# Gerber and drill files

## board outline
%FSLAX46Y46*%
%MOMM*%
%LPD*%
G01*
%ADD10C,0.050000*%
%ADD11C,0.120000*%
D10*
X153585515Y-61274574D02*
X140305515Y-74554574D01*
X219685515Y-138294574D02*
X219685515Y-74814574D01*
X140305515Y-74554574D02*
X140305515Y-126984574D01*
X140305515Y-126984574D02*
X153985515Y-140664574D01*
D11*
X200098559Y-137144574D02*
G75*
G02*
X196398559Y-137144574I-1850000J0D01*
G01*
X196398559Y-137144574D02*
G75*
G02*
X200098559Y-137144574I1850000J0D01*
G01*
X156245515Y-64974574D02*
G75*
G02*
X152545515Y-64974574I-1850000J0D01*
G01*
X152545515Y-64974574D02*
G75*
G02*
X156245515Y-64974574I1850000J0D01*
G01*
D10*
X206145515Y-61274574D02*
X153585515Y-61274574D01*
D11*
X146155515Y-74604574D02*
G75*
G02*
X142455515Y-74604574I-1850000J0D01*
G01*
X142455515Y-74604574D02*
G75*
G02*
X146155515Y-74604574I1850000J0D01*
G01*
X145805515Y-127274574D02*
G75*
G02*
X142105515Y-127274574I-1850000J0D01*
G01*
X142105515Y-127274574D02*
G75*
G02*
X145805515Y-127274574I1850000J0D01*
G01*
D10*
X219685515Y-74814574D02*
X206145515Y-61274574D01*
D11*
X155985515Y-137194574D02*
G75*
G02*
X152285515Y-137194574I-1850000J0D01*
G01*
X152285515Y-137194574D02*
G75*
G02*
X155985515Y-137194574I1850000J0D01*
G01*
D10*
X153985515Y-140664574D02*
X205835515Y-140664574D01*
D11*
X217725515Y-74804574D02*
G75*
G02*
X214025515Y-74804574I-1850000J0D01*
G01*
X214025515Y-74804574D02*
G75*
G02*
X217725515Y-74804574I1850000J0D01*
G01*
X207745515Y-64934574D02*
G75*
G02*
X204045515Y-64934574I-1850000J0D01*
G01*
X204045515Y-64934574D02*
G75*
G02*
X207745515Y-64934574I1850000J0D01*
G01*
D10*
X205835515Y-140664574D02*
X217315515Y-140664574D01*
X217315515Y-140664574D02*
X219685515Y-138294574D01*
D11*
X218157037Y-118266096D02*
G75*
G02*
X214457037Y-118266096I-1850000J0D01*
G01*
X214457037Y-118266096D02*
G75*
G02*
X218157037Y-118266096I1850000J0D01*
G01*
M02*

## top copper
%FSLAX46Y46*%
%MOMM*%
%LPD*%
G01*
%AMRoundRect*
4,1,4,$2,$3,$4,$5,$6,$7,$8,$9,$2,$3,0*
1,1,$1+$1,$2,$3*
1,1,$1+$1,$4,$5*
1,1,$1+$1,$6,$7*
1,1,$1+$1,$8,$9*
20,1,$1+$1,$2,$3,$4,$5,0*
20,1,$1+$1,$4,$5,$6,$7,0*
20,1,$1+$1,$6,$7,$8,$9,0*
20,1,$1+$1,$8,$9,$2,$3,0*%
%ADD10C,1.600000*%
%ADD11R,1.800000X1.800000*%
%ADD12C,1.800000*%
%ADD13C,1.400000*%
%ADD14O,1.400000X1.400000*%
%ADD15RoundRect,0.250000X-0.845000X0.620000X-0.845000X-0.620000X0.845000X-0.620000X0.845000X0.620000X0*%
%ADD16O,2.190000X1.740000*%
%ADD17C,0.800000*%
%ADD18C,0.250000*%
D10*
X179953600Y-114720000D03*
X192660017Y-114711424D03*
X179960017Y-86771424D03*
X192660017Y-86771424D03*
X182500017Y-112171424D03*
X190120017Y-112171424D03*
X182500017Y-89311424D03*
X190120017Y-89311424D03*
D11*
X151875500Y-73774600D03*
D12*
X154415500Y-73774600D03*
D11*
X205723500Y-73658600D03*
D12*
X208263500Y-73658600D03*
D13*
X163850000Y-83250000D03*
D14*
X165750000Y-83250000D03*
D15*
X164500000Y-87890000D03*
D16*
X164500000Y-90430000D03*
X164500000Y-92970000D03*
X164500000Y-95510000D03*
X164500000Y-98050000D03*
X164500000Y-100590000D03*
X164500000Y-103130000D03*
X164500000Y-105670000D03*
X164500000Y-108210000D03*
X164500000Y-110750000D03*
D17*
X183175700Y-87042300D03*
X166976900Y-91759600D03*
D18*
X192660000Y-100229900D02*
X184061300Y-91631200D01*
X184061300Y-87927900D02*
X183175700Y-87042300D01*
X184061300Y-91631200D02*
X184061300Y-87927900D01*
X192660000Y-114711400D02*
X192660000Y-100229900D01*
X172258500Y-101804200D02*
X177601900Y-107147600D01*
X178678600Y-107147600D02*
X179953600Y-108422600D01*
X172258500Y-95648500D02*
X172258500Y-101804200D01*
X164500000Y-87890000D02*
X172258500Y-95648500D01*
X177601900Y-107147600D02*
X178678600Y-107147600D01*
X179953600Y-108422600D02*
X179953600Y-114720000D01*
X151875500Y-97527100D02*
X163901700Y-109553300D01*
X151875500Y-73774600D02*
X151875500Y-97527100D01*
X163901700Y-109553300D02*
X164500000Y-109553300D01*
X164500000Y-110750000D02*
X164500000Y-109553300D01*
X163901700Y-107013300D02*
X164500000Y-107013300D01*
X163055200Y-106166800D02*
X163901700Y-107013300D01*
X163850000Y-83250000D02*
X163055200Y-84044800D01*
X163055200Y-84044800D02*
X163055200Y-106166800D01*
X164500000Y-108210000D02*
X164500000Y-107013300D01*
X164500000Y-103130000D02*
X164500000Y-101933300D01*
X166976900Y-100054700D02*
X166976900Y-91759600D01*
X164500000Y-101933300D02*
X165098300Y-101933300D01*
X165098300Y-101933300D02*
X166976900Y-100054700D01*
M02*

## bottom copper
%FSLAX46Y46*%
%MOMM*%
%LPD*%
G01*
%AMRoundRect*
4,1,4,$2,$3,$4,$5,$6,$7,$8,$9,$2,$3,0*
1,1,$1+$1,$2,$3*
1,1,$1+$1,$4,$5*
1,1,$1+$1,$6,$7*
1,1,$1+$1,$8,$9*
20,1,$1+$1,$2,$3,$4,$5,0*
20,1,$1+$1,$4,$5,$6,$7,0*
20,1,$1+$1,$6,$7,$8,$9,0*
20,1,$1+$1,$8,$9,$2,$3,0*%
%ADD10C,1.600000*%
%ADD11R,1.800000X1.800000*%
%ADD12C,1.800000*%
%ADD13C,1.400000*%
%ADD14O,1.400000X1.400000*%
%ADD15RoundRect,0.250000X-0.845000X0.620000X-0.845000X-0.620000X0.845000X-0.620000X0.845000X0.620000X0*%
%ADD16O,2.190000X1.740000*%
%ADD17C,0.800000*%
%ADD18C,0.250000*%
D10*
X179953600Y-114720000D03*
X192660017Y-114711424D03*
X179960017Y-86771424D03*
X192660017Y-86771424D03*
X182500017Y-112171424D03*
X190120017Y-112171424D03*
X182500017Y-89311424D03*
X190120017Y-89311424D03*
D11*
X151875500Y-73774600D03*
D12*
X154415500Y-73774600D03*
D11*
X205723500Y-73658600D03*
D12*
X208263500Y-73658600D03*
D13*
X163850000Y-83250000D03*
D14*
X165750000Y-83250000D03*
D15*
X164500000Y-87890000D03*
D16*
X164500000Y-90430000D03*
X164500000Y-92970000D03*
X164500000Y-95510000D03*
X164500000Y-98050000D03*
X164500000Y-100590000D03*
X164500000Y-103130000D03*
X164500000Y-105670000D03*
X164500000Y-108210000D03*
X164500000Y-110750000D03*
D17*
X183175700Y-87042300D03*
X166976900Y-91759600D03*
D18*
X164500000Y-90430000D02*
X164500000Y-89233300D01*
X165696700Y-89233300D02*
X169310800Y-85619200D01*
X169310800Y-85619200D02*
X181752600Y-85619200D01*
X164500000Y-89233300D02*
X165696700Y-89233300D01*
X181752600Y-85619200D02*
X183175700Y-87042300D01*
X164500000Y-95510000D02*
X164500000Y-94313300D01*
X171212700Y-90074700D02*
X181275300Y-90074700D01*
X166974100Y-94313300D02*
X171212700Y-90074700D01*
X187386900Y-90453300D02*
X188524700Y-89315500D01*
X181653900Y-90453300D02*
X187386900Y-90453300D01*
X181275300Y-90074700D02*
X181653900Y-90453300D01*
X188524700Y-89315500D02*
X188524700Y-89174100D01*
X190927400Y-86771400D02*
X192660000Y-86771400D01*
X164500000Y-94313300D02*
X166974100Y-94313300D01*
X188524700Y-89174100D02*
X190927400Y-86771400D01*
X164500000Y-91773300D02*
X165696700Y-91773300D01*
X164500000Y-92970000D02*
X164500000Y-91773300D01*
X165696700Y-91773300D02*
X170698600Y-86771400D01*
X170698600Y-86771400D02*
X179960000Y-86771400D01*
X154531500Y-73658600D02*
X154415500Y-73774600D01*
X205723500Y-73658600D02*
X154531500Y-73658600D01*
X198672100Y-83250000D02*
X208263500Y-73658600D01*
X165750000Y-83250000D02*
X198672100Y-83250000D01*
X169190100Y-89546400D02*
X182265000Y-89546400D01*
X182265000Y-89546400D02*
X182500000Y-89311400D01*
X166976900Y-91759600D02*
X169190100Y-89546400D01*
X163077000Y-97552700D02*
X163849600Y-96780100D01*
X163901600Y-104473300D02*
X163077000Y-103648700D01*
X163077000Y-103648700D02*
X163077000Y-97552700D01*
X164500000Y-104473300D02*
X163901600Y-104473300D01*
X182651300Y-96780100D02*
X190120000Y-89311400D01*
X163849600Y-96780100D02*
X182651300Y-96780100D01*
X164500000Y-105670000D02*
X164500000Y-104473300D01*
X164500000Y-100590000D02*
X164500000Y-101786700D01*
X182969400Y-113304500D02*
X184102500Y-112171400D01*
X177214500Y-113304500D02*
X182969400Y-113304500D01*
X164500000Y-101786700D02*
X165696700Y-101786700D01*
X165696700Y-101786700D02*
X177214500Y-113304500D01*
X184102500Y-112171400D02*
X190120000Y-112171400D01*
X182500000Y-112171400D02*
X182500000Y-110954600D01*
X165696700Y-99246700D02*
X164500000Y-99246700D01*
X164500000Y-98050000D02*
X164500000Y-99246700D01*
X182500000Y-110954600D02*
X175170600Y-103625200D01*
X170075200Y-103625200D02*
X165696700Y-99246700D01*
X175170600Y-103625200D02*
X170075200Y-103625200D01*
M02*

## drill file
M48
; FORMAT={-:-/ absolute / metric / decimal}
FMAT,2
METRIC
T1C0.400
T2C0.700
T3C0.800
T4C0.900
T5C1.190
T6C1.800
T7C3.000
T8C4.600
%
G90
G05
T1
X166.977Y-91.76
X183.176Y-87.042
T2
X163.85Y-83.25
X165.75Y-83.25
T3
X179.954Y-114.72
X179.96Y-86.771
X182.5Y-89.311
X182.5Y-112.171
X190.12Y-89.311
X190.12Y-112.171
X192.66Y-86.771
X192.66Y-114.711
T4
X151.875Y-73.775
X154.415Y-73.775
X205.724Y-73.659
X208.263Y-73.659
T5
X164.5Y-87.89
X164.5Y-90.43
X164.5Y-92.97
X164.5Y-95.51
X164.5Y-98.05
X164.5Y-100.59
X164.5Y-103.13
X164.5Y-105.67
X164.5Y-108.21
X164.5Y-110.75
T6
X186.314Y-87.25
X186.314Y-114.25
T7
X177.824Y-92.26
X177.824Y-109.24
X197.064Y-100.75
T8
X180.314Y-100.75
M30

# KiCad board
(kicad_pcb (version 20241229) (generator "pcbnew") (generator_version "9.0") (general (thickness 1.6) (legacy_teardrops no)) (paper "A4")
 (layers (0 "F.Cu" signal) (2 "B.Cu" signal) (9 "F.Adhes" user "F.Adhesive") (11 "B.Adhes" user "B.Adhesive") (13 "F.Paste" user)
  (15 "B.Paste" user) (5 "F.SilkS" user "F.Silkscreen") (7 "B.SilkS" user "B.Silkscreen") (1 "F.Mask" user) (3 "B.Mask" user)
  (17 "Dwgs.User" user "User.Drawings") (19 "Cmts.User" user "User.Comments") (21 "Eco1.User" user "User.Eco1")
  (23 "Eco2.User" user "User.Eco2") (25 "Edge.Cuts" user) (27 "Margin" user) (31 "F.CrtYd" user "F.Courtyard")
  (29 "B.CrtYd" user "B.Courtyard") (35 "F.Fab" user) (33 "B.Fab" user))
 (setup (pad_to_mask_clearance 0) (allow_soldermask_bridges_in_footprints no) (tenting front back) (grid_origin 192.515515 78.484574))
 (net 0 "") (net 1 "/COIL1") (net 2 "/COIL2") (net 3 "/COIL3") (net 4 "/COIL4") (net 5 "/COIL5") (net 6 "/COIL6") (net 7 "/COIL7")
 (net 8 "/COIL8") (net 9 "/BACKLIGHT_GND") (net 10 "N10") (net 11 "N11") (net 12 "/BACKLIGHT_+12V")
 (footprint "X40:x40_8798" (layer "F.Cu") (at 186.3136 100.75 90)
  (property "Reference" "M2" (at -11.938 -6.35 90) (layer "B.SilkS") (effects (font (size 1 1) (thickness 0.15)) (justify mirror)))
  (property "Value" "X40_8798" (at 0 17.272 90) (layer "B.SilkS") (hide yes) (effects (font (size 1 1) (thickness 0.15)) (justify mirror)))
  (pad "" np_thru_hole circle (at -13.5 0 90) (size 1.8 1.8) (drill 1.8) (layers "*.Cu" "*.Mask"))
  (pad "" np_thru_hole circle (at -8.49 -8.49 90) (size 3 3) (drill 3) (layers "*.Cu" "*.Mask"))
  (pad "" np_thru_hole circle (at 0 -6 90) (size 4.6 4.6) (drill 4.6) (layers "*.Cu" "*.Mask"))
  (pad "" np_thru_hole circle (at 0 10.75 90) (size 3 3) (drill 3) (layers "*.Cu" "*.Mask"))
  (pad "" np_thru_hole circle (at 8.49 -8.49 90) (size 3 3) (drill 3) (layers "*.Cu" "*.Mask"))
  (pad "" np_thru_hole circle (at 13.5 0 90) (size 1.8 1.8) (drill 1.8) (layers "*.Cu" "*.Mask"))
  (pad "1" thru_hole circle (at -13.97 -6.36 90) (size 1.6 1.6) (drill 0.8) (layers "*.Cu" "*.Mask") (remove_unused_layers no)
   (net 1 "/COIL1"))
  (pad "2" thru_hole circle (at -13.961424 6.346417 90) (size 1.6 1.6) (drill 0.8) (layers "*.Cu" "*.Mask") (remove_unused_layers no)
   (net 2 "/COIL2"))
  (pad "3" thru_hole circle (at 13.978576 -6.353583 90) (size 1.6 1.6) (drill 0.8) (layers "*.Cu" "*.Mask") (remove_unused_layers no)
   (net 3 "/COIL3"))
  (pad "4" thru_hole circle (at 13.978576 6.346417 90) (size 1.6 1.6) (drill 0.8) (layers "*.Cu" "*.Mask") (remove_unused_layers no)
   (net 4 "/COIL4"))
  (pad "5" thru_hole circle (at -11.421424 -3.813583 90) (size 1.6 1.6) (drill 0.8) (layers "*.Cu" "*.Mask") (remove_unused_layers no)
   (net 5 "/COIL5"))
  (pad "6" thru_hole circle (at -11.421424 3.806417 90) (size 1.6 1.6) (drill 0.8) (layers "*.Cu" "*.Mask") (remove_unused_layers no)
   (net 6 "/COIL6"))
  (pad "7" thru_hole circle (at 11.438576 -3.813583 90) (size 1.6 1.6) (drill 0.8) (layers "*.Cu" "*.Mask") (remove_unused_layers no)
   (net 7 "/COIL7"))
  (pad "8" thru_hole circle (at 11.438576 3.806417 90) (size 1.6 1.6) (drill 0.8) (layers "*.Cu" "*.Mask") (remove_unused_layers no)
   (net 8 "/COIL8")))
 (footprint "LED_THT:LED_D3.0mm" (layer "F.Cu") (at 151.8755 73.7746)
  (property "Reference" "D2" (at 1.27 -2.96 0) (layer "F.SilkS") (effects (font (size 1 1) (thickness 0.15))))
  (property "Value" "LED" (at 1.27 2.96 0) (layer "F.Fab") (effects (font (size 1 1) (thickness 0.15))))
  (pad "1" thru_hole rect (at 0 0) (size 1.8 1.8) (drill 0.9) (layers "*.Cu" "*.Mask") (remove_unused_layers no) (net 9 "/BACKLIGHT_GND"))
  (pad "2" thru_hole circle (at 2.54 0) (size 1.8 1.8) (drill 0.9) (layers "*.Cu" "*.Mask") (remove_unused_layers no) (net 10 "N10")))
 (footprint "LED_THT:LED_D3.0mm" (layer "F.Cu") (at 205.7235 73.6586)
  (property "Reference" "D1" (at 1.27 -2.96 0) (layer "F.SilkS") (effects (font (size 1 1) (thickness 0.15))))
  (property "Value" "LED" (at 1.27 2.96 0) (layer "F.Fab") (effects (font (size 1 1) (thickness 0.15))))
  (pad "1" thru_hole rect (at 0 0) (size 1.8 1.8) (drill 0.9) (layers "*.Cu" "*.Mask") (remove_unused_layers no) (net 10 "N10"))
  (pad "2" thru_hole circle (at 2.54 0) (size 1.8 1.8) (drill 0.9) (layers "*.Cu" "*.Mask") (remove_unused_layers no) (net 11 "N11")))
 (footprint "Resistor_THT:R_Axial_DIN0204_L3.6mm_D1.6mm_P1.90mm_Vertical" (layer "B.Cu") (at 163.85 83.25)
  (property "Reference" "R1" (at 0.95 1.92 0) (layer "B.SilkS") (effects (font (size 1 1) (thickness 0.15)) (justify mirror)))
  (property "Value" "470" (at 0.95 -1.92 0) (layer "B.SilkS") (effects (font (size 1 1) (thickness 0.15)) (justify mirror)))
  (pad "1" thru_hole circle (at 0 0) (size 1.4 1.4) (drill 0.7) (layers "*.Cu" "*.Mask") (remove_unused_layers no)
   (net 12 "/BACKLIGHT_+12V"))
  (pad "2" thru_hole oval (at 1.9 0) (size 1.4 1.4) (drill 0.7) (layers "*.Cu" "*.Mask") (remove_unused_layers no) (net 11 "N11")))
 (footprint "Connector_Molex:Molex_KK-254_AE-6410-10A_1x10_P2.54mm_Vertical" (layer "B.Cu") (at 164.5 87.89 -90)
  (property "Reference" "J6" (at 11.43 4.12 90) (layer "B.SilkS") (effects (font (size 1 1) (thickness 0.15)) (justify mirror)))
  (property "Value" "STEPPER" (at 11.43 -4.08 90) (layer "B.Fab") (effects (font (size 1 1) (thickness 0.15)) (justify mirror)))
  (pad "1" thru_hole roundrect (at 0 0 270) (size 1.74 2.19) (drill 1.19) (layers "*.Cu" "*.Mask") (remove_unused_layers no)
   (roundrect_rratio 0.143678) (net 1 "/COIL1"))
  (pad "2" thru_hole oval (at 2.54 0 270) (size 1.74 2.19) (drill 1.19) (layers "*.Cu" "*.Mask") (remove_unused_layers no) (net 2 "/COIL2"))
  (pad "3" thru_hole oval (at 5.08 0 270) (size 1.74 2.19) (drill 1.19) (layers "*.Cu" "*.Mask") (remove_unused_layers no) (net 3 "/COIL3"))
  (pad "4" thru_hole oval (at 7.62 0 270) (size 1.74 2.19) (drill 1.19) (layers "*.Cu" "*.Mask") (remove_unused_layers no) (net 4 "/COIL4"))
  (pad "5" thru_hole oval (at 10.16 0 270) (size 1.74 2.19) (drill 1.19) (layers "*.Cu" "*.Mask") (remove_unused_layers no) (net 5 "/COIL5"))
  (pad "6" thru_hole oval (at 12.7 0 270) (size 1.74 2.19) (drill 1.19) (layers "*.Cu" "*.Mask") (remove_unused_layers no) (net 6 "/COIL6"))
  (pad "7" thru_hole oval (at 15.24 0 270) (size 1.74 2.19) (drill 1.19) (layers "*.Cu" "*.Mask") (remove_unused_layers no) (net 7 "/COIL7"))
  (pad "8" thru_hole oval (at 17.78 0 270) (size 1.74 2.19) (drill 1.19) (layers "*.Cu" "*.Mask") (remove_unused_layers no) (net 8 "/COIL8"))
  (pad "9" thru_hole oval (at 20.32 0 270) (size 1.74 2.19) (drill 1.19) (layers "*.Cu" "*.Mask") (remove_unused_layers no)
   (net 12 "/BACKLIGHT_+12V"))
  (pad "10" thru_hole oval (at 22.86 0 270) (size 1.74 2.19) (drill 1.19) (layers "*.Cu" "*.Mask") (remove_unused_layers no)
   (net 9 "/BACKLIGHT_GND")))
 (gr_line (start 153.585515 61.274574) (end 140.305515 74.554574) (stroke (width 0.05) (type solid)) (layer "Edge.Cuts"))
 (gr_line (start 219.685515 138.294574) (end 219.685515 74.814574) (stroke (width 0.05) (type solid)) (layer "Edge.Cuts"))
 (gr_line (start 140.305515 74.554574) (end 140.305515 126.984574) (stroke (width 0.05) (type solid)) (layer "Edge.Cuts"))
 (gr_line (start 140.305515 126.984574) (end 153.985515 140.664574) (stroke (width 0.05) (type solid)) (layer "Edge.Cuts"))
 (gr_circle (center 198.248559 137.144574) (end 200.098559 137.144574) (stroke (width 0.12) (type solid)) (fill no) (layer "Edge.Cuts"))
 (gr_circle (center 154.395515 64.974574) (end 156.245515 64.974574) (stroke (width 0.12) (type solid)) (fill no) (layer "Edge.Cuts"))
 (gr_line (start 206.145515 61.274574) (end 153.585515 61.274574) (stroke (width 0.05) (type solid)) (layer "Edge.Cuts"))
 (gr_circle (center 144.305515 74.604574) (end 146.155515 74.604574) (stroke (width 0.12) (type solid)) (fill no) (layer "Edge.Cuts"))
 (gr_circle (center 143.955515 127.274574) (end 145.805515 127.274574) (stroke (width 0.12) (type solid)) (fill no) (layer "Edge.Cuts"))
 (gr_line (start 219.685515 74.814574) (end 206.145515 61.274574) (stroke (width 0.05) (type solid)) (layer "Edge.Cuts"))
 (gr_circle (center 154.135515 137.194574) (end 155.985515 137.194574) (stroke (width 0.12) (type solid)) (fill no) (layer "Edge.Cuts"))
 (gr_line (start 153.985515 140.664574) (end 205.835515 140.664574) (stroke (width 0.05) (type solid)) (layer "Edge.Cuts"))
 (gr_circle (center 215.875515 74.804574) (end 217.725515 74.804574) (stroke (width 0.12) (type solid)) (fill no) (layer "Edge.Cuts"))
 (gr_circle (center 205.895515 64.934574) (end 207.745515 64.934574) (stroke (width 0.12) (type solid)) (fill no) (layer "Edge.Cuts"))
 (gr_line (start 205.835515 140.664574) (end 217.315515 140.664574) (stroke (width 0.05) (type solid)) (layer "Edge.Cuts"))
 (gr_line (start 217.315515 140.664574) (end 219.685515 138.294574) (stroke (width 0.05) (type solid)) (layer "Edge.Cuts"))
 (gr_circle (center 216.307037 118.266096) (end 218.157037 118.266096) (stroke (width 0.12) (type solid)) (fill no) (layer "Edge.Cuts"))
 (segment (start 192.66 100.2299) (end 184.0613 91.6312) (width 0.25) (layer "F.Cu") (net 2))
 (segment (start 184.0613 87.9279) (end 183.1757 87.0423) (width 0.25) (layer "F.Cu") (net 2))
 (segment (start 184.0613 91.6312) (end 184.0613 87.9279) (width 0.25) (layer "F.Cu") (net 2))
 (segment (start 192.66 114.7114) (end 192.66 100.2299) (width 0.25) (layer "F.Cu") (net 2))
 (via (at 183.1757 87.0423) (size 0.8) (drill 0.4) (layers "F.Cu" "B.Cu") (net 2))
 (segment (start 164.5 90.43) (end 164.5 89.2333) (width 0.25) (layer "B.Cu") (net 2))
 (segment (start 165.6967 89.2333) (end 169.3108 85.6192) (width 0.25) (layer "B.Cu") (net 2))
 (segment (start 169.3108 85.6192) (end 181.7526 85.6192) (width 0.25) (layer "B.Cu") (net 2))
 (segment (start 164.5 89.2333) (end 165.6967 89.2333) (width 0.25) (layer "B.Cu") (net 2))
 (segment (start 181.7526 85.6192) (end 183.1757 87.0423) (width 0.25) (layer "B.Cu") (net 2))
 (segment (start 172.2585 101.8042) (end 177.6019 107.1476) (width 0.25) (layer "F.Cu") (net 1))
 (segment (start 178.6786 107.1476) (end 179.9536 108.4226) (width 0.25) (layer "F.Cu") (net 1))
 (segment (start 172.2585 95.6485) (end 172.2585 101.8042) (width 0.25) (layer "F.Cu") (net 1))
 (segment (start 164.5 87.89) (end 172.2585 95.6485) (width 0.25) (layer "F.Cu") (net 1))
 (segment (start 177.6019 107.1476) (end 178.6786 107.1476) (width 0.25) (layer "F.Cu") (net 1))
 (segment (start 179.9536 108.4226) (end 179.9536 114.72) (width 0.25) (layer "F.Cu") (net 1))
 (segment (start 164.5 95.51) (end 164.5 94.3133) (width 0.25) (layer "B.Cu") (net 4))
 (segment (start 171.2127 90.0747) (end 181.2753 90.0747) (width 0.25) (layer "B.Cu") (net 4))
 (segment (start 166.9741 94.3133) (end 171.2127 90.0747) (width 0.25) (layer "B.Cu") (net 4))
 (segment (start 187.3869 90.4533) (end 188.5247 89.3155) (width 0.25) (layer "B.Cu") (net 4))
 (segment (start 181.6539 90.4533) (end 187.3869 90.4533) (width 0.25) (layer "B.Cu") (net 4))
 (segment (start 181.2753 90.0747) (end 181.6539 90.4533) (width 0.25) (layer "B.Cu") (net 4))
 (segment (start 188.5247 89.3155) (end 188.5247 89.1741) (width 0.25) (layer "B.Cu") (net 4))
 (segment (start 190.9274 86.7714) (end 192.66 86.7714) (width 0.25) (layer "B.Cu") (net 4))
 (segment (start 164.5 94.3133) (end 166.9741 94.3133) (width 0.25) (layer "B.Cu") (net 4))
 (segment (start 188.5247 89.1741) (end 190.9274 86.7714) (width 0.25) (layer "B.Cu") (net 4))
 (segment (start 164.5 91.7733) (end 165.6967 91.7733) (width 0.25) (layer "B.Cu") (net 3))
 (segment (start 164.5 92.97) (end 164.5 91.7733) (width 0.25) (layer "B.Cu") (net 3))
 (segment (start 165.6967 91.7733) (end 170.6986 86.7714) (width 0.25) (layer "B.Cu") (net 3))
 (segment (start 170.6986 86.7714) (end 179.96 86.7714) (width 0.25) (layer "B.Cu") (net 3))
 (segment (start 154.5315 73.6586) (end 154.4155 73.7746) (width 0.25) (layer "B.Cu") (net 10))
 (segment (start 205.7235 73.6586) (end 154.5315 73.6586) (width 0.25) (layer "B.Cu") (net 10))
 (segment (start 198.6721 83.25) (end 208.2635 73.6586) (width 0.25) (layer "B.Cu") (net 11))
 (segment (start 165.75 83.25) (end 198.6721 83.25) (width 0.25) (layer "B.Cu") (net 11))
 (segment (start 151.8755 97.5271) (end 163.9017 109.5533) (width 0.25) (layer "F.Cu") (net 9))
 (segment (start 151.8755 73.7746) (end 151.8755 97.5271) (width 0.25) (layer "F.Cu") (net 9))
 (segment (start 163.9017 109.5533) (end 164.5 109.5533) (width 0.25) (layer "F.Cu") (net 9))
 (segment (start 164.5 110.75) (end 164.5 109.5533) (width 0.25) (layer "F.Cu") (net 9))
 (segment (start 163.9017 107.0133) (end 164.5 107.0133) (width 0.25) (layer "F.Cu") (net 12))
 (segment (start 163.0552 106.1668) (end 163.9017 107.0133) (width 0.25) (layer "F.Cu") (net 12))
 (segment (start 163.85 83.25) (end 163.0552 84.0448) (width 0.25) (layer "F.Cu") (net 12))
 (segment (start 163.0552 84.0448) (end 163.0552 106.1668) (width 0.25) (layer "F.Cu") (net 12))
 (segment (start 164.5 108.21) (end 164.5 107.0133) (width 0.25) (layer "F.Cu") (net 12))
 (segment (start 164.5 103.13) (end 164.5 101.9333) (width 0.25) (layer "F.Cu") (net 7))
 (segment (start 166.9769 100.0547) (end 166.9769 91.7596) (width 0.25) (layer "F.Cu") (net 7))
 (segment (start 164.5 101.9333) (end 165.0983 101.9333) (width 0.25) (layer "F.Cu") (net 7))
 (segment (start 165.0983 101.9333) (end 166.9769 100.0547) (width 0.25) (layer "F.Cu") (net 7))
 (via (at 166.9769 91.7596) (size 0.8) (drill 0.4) (layers "F.Cu" "B.Cu") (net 7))
 (segment (start 169.1901 89.5464) (end 182.265 89.5464) (width 0.25) (layer "B.Cu") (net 7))
 (segment (start 182.265 89.5464) (end 182.5 89.3114) (width 0.25) (layer "B.Cu") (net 7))
 (segment (start 166.9769 91.7596) (end 169.1901 89.5464) (width 0.25) (layer "B.Cu") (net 7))
 (segment (start 163.077 97.5527) (end 163.8496 96.7801) (width 0.25) (layer "B.Cu") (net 8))
 (segment (start 163.9016 104.4733) (end 163.077 103.6487) (width 0.25) (layer "B.Cu") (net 8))
 (segment (start 163.077 103.6487) (end 163.077 97.5527) (width 0.25) (layer "B.Cu") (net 8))
 (segment (start 164.5 104.4733) (end 163.9016 104.4733) (width 0.25) (layer "B.Cu") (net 8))
 (segment (start 182.6513 96.7801) (end 190.12 89.3114) (width 0.25) (layer "B.Cu") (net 8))
 (segment (start 163.8496 96.7801) (end 182.6513 96.7801) (width 0.25) (layer "B.Cu") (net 8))
 (segment (start 164.5 105.67) (end 164.5 104.4733) (width 0.25) (layer "B.Cu") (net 8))
 (segment (start 164.5 100.59) (end 164.5 101.7867) (width 0.25) (layer "B.Cu") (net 6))
 (segment (start 182.9694 113.3045) (end 184.1025 112.1714) (width 0.25) (layer "B.Cu") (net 6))
 (segment (start 177.2145 113.3045) (end 182.9694 113.3045) (width 0.25) (layer "B.Cu") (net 6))
 (segment (start 164.5 101.7867) (end 165.6967 101.7867) (width 0.25) (layer "B.Cu") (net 6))
 (segment (start 165.6967 101.7867) (end 177.2145 113.3045) (width 0.25) (layer "B.Cu") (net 6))
 (segment (start 184.1025 112.1714) (end 190.12 112.1714) (width 0.25) (layer "B.Cu") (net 6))
 (segment (start 182.5 112.1714) (end 182.5 110.9546) (width 0.25) (layer "B.Cu") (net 5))
 (segment (start 165.6967 99.2467) (end 164.5 99.2467) (width 0.25) (layer "B.Cu") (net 5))
 (segment (start 164.5 98.05) (end 164.5 99.2467) (width 0.25) (layer "B.Cu") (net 5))
 (segment (start 182.5 110.9546) (end 175.1706 103.6252) (width 0.25) (layer "B.Cu") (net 5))
 (segment (start 170.0752 103.6252) (end 165.6967 99.2467) (width 0.25) (layer "B.Cu") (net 5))
 (segment (start 175.1706 103.6252) (end 170.0752 103.6252) (width 0.25) (layer "B.Cu") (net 5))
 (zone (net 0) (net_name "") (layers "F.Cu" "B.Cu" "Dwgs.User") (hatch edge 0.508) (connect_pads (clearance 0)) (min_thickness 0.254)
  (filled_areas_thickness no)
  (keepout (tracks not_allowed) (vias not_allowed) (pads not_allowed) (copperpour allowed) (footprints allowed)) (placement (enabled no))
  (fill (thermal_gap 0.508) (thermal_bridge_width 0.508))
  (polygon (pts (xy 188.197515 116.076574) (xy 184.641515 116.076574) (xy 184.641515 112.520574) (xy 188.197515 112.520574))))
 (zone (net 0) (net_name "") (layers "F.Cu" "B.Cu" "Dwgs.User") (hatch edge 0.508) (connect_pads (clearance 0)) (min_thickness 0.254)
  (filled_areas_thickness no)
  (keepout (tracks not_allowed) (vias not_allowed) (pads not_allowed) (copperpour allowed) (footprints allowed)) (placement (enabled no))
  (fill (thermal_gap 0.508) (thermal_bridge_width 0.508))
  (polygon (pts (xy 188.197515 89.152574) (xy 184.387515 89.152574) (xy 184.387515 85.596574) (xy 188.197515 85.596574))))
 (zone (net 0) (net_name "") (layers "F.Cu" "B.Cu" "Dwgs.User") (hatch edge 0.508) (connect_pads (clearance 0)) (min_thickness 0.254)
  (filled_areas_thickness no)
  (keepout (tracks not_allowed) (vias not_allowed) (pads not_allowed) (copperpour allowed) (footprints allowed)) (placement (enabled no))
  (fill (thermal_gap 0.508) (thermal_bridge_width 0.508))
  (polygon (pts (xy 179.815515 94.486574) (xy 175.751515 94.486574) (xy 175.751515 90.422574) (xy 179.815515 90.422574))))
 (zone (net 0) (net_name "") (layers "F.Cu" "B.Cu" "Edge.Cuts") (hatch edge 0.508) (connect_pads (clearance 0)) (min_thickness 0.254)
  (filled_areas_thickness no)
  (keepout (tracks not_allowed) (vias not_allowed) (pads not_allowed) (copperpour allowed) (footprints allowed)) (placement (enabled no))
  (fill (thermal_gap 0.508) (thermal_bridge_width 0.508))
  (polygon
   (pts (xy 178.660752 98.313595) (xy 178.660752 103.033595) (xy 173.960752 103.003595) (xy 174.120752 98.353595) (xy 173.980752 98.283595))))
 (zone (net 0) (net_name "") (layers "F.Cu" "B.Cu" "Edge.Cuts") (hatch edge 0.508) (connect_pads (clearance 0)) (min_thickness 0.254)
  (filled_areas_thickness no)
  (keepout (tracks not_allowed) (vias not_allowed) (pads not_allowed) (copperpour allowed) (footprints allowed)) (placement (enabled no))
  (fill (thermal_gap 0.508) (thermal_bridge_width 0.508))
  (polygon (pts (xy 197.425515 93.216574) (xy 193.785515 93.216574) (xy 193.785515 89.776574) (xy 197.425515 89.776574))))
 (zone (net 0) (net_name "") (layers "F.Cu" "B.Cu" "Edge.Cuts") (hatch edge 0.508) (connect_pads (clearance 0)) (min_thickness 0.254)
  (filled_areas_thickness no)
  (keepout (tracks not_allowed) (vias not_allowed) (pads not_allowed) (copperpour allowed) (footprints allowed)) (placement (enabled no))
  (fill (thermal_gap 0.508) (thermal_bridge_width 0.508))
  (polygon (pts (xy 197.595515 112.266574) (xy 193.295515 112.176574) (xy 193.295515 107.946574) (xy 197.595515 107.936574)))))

